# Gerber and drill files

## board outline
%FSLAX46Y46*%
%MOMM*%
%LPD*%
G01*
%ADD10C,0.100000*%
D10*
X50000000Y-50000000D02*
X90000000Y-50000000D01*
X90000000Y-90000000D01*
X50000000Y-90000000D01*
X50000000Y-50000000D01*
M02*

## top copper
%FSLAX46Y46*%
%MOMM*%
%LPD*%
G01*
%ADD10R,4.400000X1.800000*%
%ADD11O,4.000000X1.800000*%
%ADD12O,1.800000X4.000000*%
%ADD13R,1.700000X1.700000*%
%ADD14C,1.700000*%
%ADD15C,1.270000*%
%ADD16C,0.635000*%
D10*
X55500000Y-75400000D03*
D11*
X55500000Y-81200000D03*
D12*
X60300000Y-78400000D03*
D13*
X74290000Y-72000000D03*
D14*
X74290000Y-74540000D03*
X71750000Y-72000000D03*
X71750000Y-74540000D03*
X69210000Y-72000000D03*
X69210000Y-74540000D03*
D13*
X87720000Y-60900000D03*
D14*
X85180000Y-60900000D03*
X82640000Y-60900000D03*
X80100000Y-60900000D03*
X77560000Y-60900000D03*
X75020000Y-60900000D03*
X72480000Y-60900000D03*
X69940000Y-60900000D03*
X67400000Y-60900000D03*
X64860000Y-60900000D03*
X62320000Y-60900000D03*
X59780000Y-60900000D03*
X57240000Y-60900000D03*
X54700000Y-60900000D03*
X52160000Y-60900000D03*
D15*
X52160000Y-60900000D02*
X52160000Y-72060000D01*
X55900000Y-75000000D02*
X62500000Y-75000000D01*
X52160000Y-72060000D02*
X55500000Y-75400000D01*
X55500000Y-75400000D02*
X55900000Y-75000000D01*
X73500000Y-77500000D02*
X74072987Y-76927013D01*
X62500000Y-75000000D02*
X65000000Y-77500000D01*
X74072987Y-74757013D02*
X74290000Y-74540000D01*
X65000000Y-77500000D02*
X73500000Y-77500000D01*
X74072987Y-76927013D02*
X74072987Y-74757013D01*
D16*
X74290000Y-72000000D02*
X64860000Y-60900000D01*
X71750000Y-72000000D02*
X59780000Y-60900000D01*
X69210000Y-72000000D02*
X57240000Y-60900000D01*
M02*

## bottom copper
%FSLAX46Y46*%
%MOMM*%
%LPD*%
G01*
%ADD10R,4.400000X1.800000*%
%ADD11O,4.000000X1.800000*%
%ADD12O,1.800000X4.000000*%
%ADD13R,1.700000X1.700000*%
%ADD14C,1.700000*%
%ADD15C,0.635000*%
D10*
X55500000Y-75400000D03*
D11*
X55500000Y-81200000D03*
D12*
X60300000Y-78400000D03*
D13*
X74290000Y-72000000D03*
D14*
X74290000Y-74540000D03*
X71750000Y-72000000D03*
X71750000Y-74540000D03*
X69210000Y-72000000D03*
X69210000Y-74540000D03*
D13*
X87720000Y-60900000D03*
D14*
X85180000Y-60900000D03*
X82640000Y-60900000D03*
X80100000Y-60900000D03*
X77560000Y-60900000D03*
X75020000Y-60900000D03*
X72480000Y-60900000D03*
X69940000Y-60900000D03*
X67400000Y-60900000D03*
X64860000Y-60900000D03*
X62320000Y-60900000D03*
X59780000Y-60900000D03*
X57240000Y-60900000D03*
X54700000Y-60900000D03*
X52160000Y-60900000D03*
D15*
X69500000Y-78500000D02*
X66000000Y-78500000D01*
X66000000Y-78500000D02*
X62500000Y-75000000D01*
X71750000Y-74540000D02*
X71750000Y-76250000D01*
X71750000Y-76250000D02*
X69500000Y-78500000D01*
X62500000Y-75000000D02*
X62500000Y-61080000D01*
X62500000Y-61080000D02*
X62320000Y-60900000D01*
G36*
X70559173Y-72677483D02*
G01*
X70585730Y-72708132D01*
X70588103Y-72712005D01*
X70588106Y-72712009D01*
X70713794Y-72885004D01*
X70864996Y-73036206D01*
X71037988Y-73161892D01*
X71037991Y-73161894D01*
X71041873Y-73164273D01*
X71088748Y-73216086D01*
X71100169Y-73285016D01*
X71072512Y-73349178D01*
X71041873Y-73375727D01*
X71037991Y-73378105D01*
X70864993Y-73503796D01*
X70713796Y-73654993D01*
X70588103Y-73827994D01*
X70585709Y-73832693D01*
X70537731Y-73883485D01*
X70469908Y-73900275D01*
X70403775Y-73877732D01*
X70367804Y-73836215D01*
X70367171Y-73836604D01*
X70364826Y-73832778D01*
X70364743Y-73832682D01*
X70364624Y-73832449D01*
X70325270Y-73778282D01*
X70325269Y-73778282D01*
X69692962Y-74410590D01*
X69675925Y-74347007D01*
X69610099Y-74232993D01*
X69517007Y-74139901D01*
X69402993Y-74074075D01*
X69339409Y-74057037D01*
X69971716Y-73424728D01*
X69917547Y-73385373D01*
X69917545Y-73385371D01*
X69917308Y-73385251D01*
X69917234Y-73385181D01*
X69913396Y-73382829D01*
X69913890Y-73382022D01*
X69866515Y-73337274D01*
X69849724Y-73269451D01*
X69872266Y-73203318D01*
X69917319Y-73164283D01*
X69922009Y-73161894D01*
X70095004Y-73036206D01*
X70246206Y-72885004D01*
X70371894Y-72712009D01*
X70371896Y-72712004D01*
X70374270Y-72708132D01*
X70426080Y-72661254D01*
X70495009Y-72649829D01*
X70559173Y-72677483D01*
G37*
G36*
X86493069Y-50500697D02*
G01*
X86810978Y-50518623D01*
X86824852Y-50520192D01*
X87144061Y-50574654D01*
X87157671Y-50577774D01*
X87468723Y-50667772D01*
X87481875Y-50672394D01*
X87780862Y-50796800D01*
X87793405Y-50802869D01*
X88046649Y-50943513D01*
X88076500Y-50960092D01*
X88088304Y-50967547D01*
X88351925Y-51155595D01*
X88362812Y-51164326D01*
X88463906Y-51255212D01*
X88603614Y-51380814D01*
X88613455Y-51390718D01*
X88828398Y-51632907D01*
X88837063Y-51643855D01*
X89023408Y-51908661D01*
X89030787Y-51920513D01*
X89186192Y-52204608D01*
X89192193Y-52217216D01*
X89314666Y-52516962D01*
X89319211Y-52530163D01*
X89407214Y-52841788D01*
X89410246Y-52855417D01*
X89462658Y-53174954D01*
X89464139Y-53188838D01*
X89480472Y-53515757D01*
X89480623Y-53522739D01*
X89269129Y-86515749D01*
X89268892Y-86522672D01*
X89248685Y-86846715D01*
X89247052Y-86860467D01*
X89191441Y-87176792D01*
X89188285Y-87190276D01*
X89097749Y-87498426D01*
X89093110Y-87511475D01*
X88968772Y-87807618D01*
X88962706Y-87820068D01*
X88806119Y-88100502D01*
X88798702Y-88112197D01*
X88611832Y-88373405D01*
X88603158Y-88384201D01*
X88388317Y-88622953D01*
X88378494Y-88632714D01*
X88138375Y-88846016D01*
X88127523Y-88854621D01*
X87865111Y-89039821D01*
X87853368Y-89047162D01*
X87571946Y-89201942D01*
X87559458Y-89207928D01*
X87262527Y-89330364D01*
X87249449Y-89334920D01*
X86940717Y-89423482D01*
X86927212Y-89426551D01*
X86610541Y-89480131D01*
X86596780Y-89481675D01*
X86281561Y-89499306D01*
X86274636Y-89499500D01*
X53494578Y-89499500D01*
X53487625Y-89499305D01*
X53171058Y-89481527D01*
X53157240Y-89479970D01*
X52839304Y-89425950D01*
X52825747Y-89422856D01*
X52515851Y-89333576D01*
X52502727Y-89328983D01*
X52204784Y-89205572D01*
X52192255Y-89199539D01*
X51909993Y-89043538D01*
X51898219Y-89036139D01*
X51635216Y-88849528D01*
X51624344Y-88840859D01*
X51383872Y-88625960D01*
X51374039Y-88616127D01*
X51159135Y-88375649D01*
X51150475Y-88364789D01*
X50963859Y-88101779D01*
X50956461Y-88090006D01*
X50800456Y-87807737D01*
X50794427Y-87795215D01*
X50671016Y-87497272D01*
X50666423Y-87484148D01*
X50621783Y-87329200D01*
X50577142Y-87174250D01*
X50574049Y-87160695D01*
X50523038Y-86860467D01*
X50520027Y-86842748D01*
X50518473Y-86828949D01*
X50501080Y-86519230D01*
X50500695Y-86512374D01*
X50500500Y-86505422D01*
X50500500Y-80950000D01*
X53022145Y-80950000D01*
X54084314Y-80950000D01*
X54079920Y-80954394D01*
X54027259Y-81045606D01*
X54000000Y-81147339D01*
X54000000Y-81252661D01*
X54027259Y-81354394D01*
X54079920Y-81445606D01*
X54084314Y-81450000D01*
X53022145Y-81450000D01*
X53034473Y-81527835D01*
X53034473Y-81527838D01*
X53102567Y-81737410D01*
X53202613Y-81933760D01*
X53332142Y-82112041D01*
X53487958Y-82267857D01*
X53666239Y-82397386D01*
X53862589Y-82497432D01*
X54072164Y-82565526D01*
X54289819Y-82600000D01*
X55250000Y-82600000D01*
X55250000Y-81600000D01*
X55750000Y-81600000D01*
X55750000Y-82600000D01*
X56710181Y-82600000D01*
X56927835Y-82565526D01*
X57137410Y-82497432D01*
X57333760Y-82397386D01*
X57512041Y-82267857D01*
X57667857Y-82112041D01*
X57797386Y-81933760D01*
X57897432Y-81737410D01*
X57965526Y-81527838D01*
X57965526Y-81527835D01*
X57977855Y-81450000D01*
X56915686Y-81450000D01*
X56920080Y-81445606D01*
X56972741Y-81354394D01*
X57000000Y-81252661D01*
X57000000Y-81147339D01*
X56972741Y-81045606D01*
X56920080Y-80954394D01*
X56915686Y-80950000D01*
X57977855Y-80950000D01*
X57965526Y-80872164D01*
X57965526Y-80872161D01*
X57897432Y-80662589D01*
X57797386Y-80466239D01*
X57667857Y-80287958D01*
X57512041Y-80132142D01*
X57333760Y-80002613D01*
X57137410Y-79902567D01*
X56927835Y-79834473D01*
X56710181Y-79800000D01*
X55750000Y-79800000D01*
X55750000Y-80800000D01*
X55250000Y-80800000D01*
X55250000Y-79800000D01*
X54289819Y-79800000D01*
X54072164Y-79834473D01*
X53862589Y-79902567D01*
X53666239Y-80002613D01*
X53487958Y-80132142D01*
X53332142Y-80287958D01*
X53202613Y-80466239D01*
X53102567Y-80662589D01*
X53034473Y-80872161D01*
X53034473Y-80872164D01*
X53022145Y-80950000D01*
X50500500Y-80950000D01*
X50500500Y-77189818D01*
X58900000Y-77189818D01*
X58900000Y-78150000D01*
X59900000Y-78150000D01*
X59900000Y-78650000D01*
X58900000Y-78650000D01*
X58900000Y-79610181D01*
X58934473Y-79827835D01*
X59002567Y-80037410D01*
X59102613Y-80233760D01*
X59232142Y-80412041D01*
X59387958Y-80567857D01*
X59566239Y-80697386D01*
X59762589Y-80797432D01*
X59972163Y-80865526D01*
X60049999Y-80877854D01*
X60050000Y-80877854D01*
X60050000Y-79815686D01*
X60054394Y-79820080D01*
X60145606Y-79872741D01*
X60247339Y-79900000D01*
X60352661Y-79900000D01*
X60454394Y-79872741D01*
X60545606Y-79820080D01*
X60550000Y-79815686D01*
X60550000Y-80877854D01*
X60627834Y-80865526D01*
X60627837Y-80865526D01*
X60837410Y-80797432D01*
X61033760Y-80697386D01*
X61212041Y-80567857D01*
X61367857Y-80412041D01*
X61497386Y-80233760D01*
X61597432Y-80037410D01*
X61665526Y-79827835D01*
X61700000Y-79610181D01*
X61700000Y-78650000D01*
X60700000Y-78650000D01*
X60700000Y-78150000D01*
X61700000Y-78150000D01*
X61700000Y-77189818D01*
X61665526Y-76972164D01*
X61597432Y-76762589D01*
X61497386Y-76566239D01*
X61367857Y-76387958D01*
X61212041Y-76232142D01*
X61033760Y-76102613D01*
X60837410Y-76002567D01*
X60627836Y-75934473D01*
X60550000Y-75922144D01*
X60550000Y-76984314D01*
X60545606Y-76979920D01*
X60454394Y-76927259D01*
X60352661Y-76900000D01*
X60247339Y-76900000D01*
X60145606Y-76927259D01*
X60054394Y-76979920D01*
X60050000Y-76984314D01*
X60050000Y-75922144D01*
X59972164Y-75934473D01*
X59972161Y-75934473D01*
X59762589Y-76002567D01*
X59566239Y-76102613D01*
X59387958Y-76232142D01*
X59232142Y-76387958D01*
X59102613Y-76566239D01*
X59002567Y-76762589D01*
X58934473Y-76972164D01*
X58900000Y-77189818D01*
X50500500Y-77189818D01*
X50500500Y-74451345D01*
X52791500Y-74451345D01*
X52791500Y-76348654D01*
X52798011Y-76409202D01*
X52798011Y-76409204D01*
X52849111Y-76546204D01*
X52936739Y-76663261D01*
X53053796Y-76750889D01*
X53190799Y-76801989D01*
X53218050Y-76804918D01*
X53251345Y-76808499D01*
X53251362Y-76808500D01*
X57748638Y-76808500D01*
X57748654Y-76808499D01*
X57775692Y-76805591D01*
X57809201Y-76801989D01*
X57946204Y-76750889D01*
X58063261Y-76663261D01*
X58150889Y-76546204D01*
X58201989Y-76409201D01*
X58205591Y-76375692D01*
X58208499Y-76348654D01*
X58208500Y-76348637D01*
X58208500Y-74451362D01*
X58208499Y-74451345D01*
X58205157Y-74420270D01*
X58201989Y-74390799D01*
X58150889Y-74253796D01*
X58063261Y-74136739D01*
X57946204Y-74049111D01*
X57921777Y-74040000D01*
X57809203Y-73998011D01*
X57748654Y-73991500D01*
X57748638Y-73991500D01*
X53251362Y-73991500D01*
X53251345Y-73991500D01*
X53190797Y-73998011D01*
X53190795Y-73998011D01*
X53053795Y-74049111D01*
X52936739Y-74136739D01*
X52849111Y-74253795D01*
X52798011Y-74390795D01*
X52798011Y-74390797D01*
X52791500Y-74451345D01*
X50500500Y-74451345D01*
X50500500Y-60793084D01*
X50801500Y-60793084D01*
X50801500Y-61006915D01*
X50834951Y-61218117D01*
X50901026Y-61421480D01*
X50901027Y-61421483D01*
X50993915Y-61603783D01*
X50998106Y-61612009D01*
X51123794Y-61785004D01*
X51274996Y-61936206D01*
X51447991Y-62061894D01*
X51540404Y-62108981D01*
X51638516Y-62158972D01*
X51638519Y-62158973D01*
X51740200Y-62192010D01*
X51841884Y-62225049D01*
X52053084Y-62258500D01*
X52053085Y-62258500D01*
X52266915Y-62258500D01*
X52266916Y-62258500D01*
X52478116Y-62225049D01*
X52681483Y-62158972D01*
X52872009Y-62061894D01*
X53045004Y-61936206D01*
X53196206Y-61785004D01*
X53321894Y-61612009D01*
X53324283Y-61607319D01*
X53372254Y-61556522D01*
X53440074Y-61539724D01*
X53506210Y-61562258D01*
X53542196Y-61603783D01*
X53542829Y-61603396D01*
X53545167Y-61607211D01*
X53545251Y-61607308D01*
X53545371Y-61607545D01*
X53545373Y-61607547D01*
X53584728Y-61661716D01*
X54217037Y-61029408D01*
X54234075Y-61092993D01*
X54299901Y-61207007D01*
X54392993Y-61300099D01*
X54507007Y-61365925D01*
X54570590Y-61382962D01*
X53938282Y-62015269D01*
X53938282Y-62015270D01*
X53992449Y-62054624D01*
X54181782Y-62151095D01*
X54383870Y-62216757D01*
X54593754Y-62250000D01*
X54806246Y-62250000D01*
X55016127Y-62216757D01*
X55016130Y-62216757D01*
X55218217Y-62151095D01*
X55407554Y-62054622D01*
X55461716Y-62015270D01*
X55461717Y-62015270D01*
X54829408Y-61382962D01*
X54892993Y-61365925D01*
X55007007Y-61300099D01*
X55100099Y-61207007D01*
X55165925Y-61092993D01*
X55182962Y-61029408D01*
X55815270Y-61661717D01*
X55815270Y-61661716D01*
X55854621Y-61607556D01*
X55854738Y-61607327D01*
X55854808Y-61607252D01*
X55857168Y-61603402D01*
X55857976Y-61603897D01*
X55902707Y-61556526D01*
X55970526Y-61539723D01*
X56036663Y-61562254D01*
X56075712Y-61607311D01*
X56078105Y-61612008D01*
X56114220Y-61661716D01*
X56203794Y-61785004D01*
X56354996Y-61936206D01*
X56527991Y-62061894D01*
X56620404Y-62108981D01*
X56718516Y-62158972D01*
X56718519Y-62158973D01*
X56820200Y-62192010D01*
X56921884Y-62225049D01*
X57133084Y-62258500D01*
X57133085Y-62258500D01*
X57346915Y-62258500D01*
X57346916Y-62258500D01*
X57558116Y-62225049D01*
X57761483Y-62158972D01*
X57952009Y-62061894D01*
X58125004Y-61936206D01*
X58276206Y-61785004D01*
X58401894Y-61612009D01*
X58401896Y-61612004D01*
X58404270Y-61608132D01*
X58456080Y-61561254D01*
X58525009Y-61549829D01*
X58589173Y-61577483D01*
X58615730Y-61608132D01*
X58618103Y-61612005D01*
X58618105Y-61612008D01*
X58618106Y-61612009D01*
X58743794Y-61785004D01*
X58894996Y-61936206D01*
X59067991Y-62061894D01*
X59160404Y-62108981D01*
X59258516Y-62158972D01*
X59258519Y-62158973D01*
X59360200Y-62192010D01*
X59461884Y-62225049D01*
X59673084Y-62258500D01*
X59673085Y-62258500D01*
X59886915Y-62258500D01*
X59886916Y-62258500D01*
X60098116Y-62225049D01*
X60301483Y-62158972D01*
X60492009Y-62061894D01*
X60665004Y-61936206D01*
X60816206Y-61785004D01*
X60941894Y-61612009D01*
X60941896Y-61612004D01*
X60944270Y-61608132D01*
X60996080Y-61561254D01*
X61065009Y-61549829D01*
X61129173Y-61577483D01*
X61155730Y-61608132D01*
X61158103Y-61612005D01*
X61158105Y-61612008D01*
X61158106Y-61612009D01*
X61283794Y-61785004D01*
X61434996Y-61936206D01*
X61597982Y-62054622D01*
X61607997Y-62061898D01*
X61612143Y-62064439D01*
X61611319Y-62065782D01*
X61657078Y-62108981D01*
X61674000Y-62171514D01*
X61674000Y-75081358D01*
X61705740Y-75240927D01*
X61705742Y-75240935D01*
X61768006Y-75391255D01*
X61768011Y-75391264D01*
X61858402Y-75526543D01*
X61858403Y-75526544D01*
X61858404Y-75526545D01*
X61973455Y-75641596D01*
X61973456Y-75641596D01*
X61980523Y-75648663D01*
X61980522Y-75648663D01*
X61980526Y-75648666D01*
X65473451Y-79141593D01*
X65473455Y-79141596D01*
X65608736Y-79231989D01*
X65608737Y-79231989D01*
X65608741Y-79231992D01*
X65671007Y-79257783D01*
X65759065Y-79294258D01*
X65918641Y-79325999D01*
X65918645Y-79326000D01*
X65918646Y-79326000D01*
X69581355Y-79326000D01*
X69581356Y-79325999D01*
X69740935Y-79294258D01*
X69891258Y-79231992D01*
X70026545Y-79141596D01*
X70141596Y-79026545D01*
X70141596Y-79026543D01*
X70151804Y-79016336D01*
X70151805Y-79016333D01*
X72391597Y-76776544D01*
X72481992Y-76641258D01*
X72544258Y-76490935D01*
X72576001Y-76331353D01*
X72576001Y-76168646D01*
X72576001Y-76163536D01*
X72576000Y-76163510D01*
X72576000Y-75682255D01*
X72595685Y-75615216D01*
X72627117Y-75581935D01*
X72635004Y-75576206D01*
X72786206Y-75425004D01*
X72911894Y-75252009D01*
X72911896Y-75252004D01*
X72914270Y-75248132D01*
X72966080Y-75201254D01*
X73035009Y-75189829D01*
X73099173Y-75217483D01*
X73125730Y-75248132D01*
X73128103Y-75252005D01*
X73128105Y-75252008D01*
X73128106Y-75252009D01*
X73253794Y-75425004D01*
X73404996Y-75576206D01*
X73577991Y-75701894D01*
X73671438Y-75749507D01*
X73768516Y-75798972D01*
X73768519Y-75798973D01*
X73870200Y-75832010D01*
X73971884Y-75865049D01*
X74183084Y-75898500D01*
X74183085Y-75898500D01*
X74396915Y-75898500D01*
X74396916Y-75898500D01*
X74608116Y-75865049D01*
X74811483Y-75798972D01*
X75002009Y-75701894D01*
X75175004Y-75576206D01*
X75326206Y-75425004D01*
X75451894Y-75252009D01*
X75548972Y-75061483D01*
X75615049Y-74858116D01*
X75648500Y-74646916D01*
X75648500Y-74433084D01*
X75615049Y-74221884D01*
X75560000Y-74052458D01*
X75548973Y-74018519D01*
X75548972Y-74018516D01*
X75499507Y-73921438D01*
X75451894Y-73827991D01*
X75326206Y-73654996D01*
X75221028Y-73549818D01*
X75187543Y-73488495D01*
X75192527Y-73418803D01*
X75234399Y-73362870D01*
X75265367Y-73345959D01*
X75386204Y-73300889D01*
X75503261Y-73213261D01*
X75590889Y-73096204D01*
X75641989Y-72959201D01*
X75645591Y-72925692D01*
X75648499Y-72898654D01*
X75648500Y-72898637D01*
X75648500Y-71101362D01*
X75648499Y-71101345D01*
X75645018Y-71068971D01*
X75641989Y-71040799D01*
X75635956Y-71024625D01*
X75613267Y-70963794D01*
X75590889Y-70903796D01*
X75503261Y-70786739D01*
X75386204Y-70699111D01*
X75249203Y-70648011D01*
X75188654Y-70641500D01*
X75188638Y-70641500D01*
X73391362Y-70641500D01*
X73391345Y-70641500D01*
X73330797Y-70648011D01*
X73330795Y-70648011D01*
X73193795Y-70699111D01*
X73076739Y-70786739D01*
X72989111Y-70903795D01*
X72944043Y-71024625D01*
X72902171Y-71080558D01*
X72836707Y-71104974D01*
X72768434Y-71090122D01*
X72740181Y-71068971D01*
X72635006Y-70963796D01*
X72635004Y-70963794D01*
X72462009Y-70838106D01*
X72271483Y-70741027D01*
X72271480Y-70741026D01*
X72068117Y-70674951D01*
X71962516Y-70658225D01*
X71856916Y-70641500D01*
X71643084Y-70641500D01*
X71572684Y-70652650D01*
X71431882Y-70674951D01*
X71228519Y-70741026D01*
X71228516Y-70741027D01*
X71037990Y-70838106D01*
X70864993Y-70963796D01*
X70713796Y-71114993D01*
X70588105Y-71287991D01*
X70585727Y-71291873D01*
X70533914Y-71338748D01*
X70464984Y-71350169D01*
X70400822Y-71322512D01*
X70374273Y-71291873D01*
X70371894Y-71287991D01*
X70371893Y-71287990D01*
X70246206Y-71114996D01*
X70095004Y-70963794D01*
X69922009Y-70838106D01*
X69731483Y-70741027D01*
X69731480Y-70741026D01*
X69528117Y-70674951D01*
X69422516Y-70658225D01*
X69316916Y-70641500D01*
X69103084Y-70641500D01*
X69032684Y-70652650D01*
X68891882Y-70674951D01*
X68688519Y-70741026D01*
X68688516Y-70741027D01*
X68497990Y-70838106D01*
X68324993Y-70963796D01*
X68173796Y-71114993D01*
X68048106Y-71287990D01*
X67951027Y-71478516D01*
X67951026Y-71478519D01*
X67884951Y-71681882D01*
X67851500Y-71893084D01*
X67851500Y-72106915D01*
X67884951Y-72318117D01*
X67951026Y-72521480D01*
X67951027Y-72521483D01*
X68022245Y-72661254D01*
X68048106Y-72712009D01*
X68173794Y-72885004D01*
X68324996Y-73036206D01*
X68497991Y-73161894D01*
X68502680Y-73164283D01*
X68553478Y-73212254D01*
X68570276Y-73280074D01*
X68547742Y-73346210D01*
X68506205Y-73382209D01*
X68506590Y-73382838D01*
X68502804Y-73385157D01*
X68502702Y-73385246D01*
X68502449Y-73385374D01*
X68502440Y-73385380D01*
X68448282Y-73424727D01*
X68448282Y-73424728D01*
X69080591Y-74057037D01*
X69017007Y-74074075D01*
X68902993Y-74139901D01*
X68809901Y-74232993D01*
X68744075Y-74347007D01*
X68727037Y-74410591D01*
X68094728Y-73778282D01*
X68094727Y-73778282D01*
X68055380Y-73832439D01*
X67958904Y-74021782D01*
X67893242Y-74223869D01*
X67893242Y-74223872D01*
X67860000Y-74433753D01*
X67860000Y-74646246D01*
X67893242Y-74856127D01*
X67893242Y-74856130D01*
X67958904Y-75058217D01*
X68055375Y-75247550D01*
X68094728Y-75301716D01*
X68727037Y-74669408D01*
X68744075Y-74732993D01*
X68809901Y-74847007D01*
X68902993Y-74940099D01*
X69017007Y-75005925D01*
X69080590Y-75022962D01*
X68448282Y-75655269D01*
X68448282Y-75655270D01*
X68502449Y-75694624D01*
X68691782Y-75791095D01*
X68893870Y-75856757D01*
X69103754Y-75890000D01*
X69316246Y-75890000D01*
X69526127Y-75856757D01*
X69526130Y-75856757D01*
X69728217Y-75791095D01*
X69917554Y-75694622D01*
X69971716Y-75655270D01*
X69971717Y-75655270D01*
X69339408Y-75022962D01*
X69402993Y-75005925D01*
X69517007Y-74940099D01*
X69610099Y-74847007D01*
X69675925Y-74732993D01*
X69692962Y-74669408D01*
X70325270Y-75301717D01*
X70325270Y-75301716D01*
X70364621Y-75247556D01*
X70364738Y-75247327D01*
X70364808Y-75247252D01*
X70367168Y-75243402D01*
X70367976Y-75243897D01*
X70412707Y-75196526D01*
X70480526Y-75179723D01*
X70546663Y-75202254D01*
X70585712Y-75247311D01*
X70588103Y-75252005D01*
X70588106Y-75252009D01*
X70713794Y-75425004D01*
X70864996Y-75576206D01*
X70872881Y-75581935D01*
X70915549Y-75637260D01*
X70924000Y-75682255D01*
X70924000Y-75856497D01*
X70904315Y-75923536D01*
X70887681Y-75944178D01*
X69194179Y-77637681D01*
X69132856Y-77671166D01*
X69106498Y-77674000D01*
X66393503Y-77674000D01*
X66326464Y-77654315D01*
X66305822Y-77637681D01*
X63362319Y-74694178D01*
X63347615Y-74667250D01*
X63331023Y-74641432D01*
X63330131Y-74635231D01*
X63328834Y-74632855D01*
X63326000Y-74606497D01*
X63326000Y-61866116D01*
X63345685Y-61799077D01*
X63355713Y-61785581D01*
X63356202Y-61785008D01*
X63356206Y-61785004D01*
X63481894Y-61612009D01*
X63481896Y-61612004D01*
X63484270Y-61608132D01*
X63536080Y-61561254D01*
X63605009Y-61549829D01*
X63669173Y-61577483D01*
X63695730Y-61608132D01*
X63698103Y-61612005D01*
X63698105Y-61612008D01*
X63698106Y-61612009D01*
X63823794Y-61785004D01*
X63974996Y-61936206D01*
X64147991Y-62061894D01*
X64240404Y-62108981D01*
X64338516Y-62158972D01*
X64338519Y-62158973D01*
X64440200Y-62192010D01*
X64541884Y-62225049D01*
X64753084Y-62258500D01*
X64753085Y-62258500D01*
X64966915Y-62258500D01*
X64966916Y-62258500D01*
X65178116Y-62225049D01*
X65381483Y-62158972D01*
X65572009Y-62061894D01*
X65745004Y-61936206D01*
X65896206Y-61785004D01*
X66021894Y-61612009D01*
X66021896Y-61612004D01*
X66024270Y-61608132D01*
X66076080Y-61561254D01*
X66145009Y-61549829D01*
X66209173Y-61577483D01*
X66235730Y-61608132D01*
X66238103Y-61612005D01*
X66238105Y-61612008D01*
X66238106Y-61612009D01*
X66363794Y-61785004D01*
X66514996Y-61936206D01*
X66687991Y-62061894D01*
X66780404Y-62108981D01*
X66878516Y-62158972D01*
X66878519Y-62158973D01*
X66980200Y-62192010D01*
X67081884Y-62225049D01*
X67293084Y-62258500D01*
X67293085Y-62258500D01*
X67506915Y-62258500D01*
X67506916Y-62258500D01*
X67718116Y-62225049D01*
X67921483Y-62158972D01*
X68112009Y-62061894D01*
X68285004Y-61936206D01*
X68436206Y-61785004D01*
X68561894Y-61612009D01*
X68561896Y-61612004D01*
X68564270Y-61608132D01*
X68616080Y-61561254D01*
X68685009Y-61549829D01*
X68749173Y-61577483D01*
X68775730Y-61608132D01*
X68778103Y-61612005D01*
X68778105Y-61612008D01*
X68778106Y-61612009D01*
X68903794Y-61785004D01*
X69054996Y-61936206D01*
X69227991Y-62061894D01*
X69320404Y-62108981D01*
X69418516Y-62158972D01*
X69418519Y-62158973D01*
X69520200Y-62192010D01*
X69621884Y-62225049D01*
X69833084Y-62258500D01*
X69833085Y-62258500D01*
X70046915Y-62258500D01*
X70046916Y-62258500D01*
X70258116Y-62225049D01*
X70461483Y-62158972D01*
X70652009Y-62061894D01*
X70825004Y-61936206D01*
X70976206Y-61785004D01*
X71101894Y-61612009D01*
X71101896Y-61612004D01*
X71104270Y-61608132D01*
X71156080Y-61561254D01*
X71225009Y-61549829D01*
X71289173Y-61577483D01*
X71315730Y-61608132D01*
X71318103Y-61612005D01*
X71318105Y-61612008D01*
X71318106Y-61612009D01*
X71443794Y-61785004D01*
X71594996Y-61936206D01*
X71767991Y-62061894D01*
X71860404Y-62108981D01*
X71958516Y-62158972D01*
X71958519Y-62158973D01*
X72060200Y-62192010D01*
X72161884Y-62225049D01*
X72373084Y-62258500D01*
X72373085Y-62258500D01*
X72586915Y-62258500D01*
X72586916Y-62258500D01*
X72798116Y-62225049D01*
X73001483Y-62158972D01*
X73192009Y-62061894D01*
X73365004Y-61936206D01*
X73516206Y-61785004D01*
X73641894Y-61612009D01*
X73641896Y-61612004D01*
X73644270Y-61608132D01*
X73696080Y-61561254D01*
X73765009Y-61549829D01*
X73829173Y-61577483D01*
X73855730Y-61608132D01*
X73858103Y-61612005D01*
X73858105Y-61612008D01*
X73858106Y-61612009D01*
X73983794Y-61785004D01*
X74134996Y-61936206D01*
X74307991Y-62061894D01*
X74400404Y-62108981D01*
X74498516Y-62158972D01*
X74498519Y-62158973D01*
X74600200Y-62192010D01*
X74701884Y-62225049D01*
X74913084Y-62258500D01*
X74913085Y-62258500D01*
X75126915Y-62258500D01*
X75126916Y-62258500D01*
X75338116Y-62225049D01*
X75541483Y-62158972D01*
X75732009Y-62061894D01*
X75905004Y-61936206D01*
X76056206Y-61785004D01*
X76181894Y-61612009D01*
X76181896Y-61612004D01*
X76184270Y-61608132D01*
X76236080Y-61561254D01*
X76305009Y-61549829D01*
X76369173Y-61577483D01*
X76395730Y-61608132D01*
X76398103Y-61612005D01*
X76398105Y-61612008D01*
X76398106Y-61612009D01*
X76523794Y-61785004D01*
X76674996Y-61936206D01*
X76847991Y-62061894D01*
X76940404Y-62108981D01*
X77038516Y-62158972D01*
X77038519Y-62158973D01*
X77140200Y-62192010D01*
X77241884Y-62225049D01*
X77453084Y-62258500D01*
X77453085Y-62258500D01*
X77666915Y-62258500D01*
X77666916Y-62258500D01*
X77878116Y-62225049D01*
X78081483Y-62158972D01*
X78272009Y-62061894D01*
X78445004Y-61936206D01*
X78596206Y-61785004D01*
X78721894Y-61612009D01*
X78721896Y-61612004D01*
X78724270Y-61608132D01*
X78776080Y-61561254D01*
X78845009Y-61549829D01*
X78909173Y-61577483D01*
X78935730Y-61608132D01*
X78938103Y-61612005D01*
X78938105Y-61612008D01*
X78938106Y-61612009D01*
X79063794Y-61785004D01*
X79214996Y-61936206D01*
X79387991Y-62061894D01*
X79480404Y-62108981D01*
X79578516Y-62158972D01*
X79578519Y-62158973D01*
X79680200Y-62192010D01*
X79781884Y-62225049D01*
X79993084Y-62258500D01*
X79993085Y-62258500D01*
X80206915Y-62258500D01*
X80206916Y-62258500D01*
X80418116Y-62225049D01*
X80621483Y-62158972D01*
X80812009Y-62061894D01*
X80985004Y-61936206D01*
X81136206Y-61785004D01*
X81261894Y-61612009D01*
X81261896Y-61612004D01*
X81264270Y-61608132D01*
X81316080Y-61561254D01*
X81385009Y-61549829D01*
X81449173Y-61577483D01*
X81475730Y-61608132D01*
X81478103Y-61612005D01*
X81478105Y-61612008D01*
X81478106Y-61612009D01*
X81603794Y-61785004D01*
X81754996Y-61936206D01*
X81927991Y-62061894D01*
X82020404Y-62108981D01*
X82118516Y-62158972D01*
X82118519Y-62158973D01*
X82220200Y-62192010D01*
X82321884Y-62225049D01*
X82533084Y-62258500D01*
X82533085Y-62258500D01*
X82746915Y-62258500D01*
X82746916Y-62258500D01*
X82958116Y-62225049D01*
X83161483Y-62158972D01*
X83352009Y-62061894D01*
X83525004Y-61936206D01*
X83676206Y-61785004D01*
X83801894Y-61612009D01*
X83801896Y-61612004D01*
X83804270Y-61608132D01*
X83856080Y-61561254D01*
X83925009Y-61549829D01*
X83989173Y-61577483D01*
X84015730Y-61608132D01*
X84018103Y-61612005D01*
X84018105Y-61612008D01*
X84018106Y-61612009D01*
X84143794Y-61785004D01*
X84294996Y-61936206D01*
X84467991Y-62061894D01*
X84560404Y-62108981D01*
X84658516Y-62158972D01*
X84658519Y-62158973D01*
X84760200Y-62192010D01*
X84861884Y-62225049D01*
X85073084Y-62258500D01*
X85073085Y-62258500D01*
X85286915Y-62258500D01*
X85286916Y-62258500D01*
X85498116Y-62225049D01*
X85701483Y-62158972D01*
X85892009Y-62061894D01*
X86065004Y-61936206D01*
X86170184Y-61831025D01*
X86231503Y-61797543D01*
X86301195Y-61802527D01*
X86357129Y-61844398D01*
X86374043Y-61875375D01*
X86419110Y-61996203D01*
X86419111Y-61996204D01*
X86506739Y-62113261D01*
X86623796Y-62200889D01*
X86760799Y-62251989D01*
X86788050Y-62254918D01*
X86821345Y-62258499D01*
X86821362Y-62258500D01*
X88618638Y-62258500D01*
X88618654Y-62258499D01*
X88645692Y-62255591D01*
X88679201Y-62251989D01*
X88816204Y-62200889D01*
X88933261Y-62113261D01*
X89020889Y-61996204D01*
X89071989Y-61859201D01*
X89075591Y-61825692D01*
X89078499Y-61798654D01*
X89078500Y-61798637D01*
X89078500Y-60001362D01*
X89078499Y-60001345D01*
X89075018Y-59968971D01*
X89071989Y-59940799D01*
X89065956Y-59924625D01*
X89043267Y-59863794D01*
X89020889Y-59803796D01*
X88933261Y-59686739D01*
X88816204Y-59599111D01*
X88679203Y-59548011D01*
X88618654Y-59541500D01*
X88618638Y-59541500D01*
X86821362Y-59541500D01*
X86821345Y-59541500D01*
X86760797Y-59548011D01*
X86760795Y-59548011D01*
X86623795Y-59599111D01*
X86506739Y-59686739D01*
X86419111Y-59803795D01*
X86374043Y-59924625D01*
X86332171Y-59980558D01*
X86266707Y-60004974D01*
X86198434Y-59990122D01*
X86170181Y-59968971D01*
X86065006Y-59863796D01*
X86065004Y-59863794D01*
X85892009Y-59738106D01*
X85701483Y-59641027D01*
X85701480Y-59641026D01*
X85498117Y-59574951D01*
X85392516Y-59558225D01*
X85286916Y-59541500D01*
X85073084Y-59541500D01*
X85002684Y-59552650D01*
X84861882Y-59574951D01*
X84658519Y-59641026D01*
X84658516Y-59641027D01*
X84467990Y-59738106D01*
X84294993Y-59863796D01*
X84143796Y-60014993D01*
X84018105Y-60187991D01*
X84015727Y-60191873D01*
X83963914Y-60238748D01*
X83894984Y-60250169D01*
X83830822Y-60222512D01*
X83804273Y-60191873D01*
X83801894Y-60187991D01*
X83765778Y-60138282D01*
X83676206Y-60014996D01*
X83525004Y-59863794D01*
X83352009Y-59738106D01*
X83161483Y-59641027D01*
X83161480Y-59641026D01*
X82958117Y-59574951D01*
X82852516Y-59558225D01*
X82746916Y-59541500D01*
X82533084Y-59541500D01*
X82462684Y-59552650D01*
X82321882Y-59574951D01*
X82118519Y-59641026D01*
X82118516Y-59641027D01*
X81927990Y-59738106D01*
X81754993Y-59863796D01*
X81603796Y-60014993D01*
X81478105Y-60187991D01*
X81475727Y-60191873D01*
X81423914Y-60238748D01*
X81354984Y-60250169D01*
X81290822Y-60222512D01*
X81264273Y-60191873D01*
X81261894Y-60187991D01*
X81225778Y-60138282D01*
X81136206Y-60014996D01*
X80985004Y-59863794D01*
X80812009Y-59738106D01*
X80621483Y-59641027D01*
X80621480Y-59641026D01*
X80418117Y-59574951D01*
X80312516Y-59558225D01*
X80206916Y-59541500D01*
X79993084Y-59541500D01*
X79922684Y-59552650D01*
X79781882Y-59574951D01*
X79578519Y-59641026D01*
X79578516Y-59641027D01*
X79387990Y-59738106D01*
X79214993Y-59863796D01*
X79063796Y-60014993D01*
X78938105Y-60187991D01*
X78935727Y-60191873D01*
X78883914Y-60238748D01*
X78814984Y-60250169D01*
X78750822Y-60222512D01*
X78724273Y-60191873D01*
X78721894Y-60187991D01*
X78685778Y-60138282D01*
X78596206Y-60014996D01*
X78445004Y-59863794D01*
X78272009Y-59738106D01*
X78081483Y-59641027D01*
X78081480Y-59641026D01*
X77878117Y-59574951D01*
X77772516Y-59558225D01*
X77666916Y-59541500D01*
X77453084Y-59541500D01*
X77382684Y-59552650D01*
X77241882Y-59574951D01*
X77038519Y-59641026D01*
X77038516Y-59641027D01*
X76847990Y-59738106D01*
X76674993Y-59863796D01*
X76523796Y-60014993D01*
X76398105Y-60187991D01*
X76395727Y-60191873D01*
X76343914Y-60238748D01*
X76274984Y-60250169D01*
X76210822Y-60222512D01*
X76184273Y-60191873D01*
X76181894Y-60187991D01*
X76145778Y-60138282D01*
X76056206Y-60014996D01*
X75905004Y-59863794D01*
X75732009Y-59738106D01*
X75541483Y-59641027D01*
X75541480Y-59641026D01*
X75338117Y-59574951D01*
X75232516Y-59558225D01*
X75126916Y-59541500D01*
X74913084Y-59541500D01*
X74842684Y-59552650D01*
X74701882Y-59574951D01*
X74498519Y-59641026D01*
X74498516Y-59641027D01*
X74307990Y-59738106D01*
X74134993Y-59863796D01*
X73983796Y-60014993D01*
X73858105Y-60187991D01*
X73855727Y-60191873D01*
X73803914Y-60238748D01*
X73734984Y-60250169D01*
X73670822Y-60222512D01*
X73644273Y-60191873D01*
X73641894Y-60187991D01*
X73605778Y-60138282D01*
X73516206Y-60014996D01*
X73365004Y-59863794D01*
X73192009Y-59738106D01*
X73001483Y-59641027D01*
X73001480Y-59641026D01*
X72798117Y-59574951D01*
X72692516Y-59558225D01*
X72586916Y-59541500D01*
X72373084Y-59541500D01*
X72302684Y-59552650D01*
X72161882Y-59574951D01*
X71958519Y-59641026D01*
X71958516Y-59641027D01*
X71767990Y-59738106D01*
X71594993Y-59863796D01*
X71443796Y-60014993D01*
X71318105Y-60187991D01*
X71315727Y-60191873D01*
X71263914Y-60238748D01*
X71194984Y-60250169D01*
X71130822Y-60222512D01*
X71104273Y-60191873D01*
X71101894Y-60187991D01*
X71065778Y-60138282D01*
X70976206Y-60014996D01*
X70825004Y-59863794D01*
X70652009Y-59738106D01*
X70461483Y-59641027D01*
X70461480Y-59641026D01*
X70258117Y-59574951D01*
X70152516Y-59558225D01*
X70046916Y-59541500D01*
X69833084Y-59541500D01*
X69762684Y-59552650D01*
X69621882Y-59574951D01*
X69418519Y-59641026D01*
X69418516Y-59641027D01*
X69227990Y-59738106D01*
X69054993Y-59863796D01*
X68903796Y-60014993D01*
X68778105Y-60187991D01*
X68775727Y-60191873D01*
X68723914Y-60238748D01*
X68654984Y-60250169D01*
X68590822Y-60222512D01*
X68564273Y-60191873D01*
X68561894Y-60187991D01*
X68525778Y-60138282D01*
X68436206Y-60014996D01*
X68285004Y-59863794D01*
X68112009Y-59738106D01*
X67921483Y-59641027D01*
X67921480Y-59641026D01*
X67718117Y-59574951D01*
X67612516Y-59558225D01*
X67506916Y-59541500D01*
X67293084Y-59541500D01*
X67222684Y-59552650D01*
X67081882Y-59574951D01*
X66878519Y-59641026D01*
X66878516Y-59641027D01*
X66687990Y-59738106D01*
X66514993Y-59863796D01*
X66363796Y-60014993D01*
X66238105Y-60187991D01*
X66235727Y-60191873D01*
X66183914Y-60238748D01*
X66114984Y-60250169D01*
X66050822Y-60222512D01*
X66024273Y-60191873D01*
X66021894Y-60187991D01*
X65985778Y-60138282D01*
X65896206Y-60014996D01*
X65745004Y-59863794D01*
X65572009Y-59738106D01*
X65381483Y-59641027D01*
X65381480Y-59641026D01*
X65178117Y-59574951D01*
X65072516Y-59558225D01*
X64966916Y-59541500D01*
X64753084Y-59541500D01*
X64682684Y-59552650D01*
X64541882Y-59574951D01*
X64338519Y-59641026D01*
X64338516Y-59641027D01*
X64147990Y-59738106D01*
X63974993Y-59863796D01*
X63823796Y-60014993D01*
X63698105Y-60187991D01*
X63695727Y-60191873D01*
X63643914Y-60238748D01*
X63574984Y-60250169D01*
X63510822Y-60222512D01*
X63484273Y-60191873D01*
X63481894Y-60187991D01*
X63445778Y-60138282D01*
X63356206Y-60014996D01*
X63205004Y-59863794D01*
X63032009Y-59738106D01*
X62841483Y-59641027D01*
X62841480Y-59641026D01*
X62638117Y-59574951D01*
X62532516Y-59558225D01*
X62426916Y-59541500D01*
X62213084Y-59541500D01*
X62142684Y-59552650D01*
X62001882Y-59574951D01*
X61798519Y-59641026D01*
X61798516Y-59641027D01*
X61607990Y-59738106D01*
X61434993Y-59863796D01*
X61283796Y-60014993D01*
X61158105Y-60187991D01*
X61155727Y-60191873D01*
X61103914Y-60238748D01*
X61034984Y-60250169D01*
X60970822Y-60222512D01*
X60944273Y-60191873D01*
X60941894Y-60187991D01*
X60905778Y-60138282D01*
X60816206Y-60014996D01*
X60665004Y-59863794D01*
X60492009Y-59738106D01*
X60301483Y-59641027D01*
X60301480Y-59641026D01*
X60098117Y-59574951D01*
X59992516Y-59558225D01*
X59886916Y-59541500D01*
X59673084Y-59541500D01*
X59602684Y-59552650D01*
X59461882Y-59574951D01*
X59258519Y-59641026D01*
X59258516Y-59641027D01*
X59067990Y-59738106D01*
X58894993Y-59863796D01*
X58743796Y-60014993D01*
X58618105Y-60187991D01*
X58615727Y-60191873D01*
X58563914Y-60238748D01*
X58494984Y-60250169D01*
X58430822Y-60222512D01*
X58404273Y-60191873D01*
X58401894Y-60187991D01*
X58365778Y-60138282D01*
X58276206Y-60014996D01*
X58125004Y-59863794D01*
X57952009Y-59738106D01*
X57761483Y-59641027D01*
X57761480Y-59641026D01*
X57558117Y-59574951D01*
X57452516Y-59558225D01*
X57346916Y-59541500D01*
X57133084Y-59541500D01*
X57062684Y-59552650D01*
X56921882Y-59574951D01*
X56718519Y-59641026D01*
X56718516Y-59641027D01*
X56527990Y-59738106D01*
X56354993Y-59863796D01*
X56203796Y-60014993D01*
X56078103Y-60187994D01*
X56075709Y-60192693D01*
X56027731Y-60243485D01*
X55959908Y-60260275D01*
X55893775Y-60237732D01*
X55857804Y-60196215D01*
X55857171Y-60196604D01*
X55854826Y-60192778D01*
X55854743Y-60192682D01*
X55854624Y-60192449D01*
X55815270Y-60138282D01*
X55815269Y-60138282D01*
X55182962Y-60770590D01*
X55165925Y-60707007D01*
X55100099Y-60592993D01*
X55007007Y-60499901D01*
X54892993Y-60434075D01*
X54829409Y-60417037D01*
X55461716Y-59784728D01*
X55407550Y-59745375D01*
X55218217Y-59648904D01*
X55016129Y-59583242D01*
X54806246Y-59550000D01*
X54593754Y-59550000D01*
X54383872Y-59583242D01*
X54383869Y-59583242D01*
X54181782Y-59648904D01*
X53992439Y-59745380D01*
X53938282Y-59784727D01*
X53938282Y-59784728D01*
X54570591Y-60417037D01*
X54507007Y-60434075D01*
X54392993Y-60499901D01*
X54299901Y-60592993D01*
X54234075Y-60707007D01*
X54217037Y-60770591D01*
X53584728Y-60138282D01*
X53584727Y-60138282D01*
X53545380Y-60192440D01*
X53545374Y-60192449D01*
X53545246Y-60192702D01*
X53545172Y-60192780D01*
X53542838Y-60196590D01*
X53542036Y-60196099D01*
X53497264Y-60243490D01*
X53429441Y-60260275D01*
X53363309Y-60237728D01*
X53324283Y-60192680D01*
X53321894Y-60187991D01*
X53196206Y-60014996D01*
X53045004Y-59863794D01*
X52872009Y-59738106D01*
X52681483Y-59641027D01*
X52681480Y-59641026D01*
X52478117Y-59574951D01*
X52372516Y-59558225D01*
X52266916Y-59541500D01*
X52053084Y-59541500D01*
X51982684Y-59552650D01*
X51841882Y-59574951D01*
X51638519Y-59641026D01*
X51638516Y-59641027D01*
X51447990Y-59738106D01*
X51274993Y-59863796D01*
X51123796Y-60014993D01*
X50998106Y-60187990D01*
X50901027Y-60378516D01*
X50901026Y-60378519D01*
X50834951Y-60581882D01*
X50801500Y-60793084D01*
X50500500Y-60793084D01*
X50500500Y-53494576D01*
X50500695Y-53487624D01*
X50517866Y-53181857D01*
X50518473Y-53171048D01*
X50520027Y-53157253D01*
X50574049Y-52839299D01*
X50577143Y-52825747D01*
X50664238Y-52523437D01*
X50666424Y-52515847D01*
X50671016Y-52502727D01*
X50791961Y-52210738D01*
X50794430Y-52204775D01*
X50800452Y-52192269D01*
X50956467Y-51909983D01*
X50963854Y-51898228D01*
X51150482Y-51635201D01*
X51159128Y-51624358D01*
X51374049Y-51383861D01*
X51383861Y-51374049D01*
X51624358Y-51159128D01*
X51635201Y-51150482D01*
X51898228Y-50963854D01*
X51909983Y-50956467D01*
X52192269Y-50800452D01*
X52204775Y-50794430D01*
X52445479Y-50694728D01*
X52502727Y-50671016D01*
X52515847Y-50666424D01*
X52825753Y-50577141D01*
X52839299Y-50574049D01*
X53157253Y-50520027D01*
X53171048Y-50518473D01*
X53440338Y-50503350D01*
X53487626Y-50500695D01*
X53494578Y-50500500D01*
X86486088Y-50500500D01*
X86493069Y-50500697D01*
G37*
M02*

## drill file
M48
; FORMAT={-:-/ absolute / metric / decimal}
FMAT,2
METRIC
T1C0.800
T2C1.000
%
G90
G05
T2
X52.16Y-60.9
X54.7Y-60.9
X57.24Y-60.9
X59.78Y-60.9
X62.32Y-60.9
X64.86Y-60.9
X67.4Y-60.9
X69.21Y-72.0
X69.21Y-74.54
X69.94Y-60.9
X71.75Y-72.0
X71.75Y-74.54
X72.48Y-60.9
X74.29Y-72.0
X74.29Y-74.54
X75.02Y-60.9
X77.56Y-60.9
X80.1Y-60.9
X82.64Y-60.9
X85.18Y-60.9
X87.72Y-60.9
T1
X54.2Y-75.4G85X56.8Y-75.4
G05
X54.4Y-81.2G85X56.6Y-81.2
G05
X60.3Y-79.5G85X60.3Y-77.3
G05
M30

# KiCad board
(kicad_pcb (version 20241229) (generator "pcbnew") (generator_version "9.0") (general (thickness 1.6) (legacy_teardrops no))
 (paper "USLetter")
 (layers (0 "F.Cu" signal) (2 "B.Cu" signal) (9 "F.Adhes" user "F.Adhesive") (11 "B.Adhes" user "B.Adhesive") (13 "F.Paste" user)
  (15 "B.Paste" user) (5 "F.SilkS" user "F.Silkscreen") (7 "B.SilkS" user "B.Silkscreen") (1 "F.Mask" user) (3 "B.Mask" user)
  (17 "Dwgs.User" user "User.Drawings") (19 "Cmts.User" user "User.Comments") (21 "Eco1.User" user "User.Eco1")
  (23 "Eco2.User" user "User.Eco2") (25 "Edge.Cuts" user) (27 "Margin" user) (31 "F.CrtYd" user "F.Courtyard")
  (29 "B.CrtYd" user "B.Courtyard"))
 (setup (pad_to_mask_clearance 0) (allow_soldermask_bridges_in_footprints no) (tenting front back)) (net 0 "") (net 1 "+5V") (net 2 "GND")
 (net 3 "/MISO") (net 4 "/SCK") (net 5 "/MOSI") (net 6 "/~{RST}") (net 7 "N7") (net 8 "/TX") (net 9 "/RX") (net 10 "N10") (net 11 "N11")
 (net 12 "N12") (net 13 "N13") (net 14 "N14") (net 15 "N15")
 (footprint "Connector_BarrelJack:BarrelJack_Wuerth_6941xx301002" (layer "F.Cu") (at 55.5 75.4)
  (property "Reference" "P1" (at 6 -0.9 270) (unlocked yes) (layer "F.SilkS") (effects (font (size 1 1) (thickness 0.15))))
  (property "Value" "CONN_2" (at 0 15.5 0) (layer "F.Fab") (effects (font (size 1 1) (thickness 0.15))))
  (pad "1" thru_hole rect (at 0 0) (size 4.4 1.8) (drill oval 3.4 0.8) (layers "*.Cu" "*.Mask") (remove_unused_layers no) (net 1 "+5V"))
  (pad "2" thru_hole oval (at 0 5.8) (size 4 1.8) (drill oval 3 0.8) (layers "*.Cu" "*.Mask") (remove_unused_layers no) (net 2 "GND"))
  (pad "3" thru_hole oval (at 4.8 3 90) (size 4 1.8) (drill oval 3 0.8) (layers "*.Cu" "*.Mask") (remove_unused_layers no) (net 2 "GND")))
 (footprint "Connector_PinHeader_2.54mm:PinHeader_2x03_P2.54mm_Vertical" (layer "F.Cu") (at 74.29 72 -90)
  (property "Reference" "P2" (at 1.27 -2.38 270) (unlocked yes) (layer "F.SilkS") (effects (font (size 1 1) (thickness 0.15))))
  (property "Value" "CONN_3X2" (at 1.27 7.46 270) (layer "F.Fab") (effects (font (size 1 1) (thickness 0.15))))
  (pad "1" thru_hole rect (at 0 0 270) (size 1.7 1.7) (drill 1) (layers "*.Cu" "*.Mask") (remove_unused_layers no) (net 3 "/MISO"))
  (pad "2" thru_hole circle (at 2.54 0 270) (size 1.7 1.7) (drill 1) (layers "*.Cu" "*.Mask") (remove_unused_layers no) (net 1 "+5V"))
  (pad "3" thru_hole circle (at 0 2.54 270) (size 1.7 1.7) (drill 1) (layers "*.Cu" "*.Mask") (remove_unused_layers no) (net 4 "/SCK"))
  (pad "4" thru_hole circle (at 2.54 2.54 270) (size 1.7 1.7) (drill 1) (layers "*.Cu" "*.Mask") (remove_unused_layers no) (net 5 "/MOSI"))
  (pad "5" thru_hole circle (at 0 5.08 270) (size 1.7 1.7) (drill 1) (layers "*.Cu" "*.Mask") (remove_unused_layers no) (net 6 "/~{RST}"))
  (pad "6" thru_hole circle (at 2.54 5.08 270) (size 1.7 1.7) (drill 1) (layers "*.Cu" "*.Mask") (remove_unused_layers no) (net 2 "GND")))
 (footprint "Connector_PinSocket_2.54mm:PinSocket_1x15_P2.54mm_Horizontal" (layer "F.Cu") (at 87.72 60.9 -90)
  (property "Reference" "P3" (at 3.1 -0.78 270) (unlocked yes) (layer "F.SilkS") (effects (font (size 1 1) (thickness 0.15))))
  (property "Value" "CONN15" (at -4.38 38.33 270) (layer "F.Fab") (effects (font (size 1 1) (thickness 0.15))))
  (pad "1" thru_hole rect (at 0 0 270) (size 1.7 1.7) (drill 1) (layers "*.Cu" "*.Mask") (remove_unused_layers no) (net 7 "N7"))
  (pad "2" thru_hole circle (at 0 2.54 270) (size 1.7 1.7) (drill 1) (layers "*.Cu" "*.Mask") (remove_unused_layers no) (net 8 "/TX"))
  (pad "3" thru_hole circle (at 0 5.08 270) (size 1.7 1.7) (drill 1) (layers "*.Cu" "*.Mask") (remove_unused_layers no) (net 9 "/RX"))
  (pad "4" thru_hole circle (at 0 7.62 270) (size 1.7 1.7) (drill 1) (layers "*.Cu" "*.Mask") (remove_unused_layers no) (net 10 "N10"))
  (pad "5" thru_hole circle (at 0 10.16 270) (size 1.7 1.7) (drill 1) (layers "*.Cu" "*.Mask") (remove_unused_layers no) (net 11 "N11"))
  (pad "6" thru_hole circle (at 0 12.7 270) (size 1.7 1.7) (drill 1) (layers "*.Cu" "*.Mask") (remove_unused_layers no) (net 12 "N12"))
  (pad "7" thru_hole circle (at 0 15.24 270) (size 1.7 1.7) (drill 1) (layers "*.Cu" "*.Mask") (remove_unused_layers no) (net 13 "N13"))
  (pad "8" thru_hole circle (at 0 17.78 270) (size 1.7 1.7) (drill 1) (layers "*.Cu" "*.Mask") (remove_unused_layers no) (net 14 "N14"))
  (pad "9" thru_hole circle (at 0 20.32 270) (size 1.7 1.7) (drill 1) (layers "*.Cu" "*.Mask") (remove_unused_layers no) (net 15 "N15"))
  (pad "10" thru_hole circle (at 0 22.86 270) (size 1.7 1.7) (drill 1) (layers "*.Cu" "*.Mask") (remove_unused_layers no) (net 3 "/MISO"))
  (pad "11" thru_hole circle (at 0 25.4 270) (size 1.7 1.7) (drill 1) (layers "*.Cu" "*.Mask") (remove_unused_layers no) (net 5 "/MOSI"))
  (pad "12" thru_hole circle (at 0 27.94 270) (size 1.7 1.7) (drill 1) (layers "*.Cu" "*.Mask") (remove_unused_layers no) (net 4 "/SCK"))
  (pad "13" thru_hole circle (at 0 30.48 270) (size 1.7 1.7) (drill 1) (layers "*.Cu" "*.Mask") (remove_unused_layers no) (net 6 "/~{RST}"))
  (pad "14" thru_hole circle (at 0 33.02 270) (size 1.7 1.7) (drill 1) (layers "*.Cu" "*.Mask") (remove_unused_layers no) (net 2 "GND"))
  (pad "15" thru_hole circle (at 0 35.56 270) (size 1.7 1.7) (drill 1) (layers "*.Cu" "*.Mask") (remove_unused_layers no) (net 1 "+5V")))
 (gr_rect (start 50 50) (end 90 90) (stroke (width 0.1) (type default)) (fill no) (layer "Edge.Cuts"))
 (segment (start 52.16 60.9) (end 52.16 72.06) (width 1.27) (layer "F.Cu") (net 1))
 (segment (start 55.9 75) (end 62.5 75) (width 1.27) (layer "F.Cu") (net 1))
 (segment (start 52.16 72.06) (end 55.5 75.4) (width 1.27) (layer "F.Cu") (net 1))
 (segment (start 55.5 75.4) (end 55.9 75) (width 1.27) (layer "F.Cu") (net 1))
 (segment (start 73.5 77.5) (end 74.072987 76.927013) (width 1.27) (layer "F.Cu") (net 1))
 (segment (start 62.5 75) (end 65 77.5) (width 1.27) (layer "F.Cu") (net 1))
 (segment (start 74.072987 74.757013) (end 74.29 74.54) (width 1.27) (layer "F.Cu") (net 1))
 (segment (start 65 77.5) (end 73.5 77.5) (width 1.27) (layer "F.Cu") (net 1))
 (segment (start 74.072987 76.927013) (end 74.072987 74.757013) (width 1.27) (layer "F.Cu") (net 1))
 (segment (start 74.29 72) (end 64.86 60.9) (width 0.635) (layer "F.Cu") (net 3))
 (segment (start 69.5 78.5) (end 66 78.5) (width 0.635) (layer "B.Cu") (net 5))
 (segment (start 66 78.5) (end 62.5 75) (width 0.635) (layer "B.Cu") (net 5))
 (segment (start 71.75 74.54) (end 71.75 76.25) (width 0.635) (layer "B.Cu") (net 5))
 (segment (start 71.75 76.25) (end 69.5 78.5) (width 0.635) (layer "B.Cu") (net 5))
 (segment (start 62.5 75) (end 62.5 61.08) (width 0.635) (layer "B.Cu") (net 5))
 (segment (start 62.5 61.08) (end 62.32 60.9) (width 0.635) (layer "B.Cu") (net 5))
 (segment (start 71.75 72) (end 59.78 60.9) (width 0.635) (layer "F.Cu") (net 4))
 (segment (start 69.21 72) (end 57.24 60.9) (width 0.635) (layer "F.Cu") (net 6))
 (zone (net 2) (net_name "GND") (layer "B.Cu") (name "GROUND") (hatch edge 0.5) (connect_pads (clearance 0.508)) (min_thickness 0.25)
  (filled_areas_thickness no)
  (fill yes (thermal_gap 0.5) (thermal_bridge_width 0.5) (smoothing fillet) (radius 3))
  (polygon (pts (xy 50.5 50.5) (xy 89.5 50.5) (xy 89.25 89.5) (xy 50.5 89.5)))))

